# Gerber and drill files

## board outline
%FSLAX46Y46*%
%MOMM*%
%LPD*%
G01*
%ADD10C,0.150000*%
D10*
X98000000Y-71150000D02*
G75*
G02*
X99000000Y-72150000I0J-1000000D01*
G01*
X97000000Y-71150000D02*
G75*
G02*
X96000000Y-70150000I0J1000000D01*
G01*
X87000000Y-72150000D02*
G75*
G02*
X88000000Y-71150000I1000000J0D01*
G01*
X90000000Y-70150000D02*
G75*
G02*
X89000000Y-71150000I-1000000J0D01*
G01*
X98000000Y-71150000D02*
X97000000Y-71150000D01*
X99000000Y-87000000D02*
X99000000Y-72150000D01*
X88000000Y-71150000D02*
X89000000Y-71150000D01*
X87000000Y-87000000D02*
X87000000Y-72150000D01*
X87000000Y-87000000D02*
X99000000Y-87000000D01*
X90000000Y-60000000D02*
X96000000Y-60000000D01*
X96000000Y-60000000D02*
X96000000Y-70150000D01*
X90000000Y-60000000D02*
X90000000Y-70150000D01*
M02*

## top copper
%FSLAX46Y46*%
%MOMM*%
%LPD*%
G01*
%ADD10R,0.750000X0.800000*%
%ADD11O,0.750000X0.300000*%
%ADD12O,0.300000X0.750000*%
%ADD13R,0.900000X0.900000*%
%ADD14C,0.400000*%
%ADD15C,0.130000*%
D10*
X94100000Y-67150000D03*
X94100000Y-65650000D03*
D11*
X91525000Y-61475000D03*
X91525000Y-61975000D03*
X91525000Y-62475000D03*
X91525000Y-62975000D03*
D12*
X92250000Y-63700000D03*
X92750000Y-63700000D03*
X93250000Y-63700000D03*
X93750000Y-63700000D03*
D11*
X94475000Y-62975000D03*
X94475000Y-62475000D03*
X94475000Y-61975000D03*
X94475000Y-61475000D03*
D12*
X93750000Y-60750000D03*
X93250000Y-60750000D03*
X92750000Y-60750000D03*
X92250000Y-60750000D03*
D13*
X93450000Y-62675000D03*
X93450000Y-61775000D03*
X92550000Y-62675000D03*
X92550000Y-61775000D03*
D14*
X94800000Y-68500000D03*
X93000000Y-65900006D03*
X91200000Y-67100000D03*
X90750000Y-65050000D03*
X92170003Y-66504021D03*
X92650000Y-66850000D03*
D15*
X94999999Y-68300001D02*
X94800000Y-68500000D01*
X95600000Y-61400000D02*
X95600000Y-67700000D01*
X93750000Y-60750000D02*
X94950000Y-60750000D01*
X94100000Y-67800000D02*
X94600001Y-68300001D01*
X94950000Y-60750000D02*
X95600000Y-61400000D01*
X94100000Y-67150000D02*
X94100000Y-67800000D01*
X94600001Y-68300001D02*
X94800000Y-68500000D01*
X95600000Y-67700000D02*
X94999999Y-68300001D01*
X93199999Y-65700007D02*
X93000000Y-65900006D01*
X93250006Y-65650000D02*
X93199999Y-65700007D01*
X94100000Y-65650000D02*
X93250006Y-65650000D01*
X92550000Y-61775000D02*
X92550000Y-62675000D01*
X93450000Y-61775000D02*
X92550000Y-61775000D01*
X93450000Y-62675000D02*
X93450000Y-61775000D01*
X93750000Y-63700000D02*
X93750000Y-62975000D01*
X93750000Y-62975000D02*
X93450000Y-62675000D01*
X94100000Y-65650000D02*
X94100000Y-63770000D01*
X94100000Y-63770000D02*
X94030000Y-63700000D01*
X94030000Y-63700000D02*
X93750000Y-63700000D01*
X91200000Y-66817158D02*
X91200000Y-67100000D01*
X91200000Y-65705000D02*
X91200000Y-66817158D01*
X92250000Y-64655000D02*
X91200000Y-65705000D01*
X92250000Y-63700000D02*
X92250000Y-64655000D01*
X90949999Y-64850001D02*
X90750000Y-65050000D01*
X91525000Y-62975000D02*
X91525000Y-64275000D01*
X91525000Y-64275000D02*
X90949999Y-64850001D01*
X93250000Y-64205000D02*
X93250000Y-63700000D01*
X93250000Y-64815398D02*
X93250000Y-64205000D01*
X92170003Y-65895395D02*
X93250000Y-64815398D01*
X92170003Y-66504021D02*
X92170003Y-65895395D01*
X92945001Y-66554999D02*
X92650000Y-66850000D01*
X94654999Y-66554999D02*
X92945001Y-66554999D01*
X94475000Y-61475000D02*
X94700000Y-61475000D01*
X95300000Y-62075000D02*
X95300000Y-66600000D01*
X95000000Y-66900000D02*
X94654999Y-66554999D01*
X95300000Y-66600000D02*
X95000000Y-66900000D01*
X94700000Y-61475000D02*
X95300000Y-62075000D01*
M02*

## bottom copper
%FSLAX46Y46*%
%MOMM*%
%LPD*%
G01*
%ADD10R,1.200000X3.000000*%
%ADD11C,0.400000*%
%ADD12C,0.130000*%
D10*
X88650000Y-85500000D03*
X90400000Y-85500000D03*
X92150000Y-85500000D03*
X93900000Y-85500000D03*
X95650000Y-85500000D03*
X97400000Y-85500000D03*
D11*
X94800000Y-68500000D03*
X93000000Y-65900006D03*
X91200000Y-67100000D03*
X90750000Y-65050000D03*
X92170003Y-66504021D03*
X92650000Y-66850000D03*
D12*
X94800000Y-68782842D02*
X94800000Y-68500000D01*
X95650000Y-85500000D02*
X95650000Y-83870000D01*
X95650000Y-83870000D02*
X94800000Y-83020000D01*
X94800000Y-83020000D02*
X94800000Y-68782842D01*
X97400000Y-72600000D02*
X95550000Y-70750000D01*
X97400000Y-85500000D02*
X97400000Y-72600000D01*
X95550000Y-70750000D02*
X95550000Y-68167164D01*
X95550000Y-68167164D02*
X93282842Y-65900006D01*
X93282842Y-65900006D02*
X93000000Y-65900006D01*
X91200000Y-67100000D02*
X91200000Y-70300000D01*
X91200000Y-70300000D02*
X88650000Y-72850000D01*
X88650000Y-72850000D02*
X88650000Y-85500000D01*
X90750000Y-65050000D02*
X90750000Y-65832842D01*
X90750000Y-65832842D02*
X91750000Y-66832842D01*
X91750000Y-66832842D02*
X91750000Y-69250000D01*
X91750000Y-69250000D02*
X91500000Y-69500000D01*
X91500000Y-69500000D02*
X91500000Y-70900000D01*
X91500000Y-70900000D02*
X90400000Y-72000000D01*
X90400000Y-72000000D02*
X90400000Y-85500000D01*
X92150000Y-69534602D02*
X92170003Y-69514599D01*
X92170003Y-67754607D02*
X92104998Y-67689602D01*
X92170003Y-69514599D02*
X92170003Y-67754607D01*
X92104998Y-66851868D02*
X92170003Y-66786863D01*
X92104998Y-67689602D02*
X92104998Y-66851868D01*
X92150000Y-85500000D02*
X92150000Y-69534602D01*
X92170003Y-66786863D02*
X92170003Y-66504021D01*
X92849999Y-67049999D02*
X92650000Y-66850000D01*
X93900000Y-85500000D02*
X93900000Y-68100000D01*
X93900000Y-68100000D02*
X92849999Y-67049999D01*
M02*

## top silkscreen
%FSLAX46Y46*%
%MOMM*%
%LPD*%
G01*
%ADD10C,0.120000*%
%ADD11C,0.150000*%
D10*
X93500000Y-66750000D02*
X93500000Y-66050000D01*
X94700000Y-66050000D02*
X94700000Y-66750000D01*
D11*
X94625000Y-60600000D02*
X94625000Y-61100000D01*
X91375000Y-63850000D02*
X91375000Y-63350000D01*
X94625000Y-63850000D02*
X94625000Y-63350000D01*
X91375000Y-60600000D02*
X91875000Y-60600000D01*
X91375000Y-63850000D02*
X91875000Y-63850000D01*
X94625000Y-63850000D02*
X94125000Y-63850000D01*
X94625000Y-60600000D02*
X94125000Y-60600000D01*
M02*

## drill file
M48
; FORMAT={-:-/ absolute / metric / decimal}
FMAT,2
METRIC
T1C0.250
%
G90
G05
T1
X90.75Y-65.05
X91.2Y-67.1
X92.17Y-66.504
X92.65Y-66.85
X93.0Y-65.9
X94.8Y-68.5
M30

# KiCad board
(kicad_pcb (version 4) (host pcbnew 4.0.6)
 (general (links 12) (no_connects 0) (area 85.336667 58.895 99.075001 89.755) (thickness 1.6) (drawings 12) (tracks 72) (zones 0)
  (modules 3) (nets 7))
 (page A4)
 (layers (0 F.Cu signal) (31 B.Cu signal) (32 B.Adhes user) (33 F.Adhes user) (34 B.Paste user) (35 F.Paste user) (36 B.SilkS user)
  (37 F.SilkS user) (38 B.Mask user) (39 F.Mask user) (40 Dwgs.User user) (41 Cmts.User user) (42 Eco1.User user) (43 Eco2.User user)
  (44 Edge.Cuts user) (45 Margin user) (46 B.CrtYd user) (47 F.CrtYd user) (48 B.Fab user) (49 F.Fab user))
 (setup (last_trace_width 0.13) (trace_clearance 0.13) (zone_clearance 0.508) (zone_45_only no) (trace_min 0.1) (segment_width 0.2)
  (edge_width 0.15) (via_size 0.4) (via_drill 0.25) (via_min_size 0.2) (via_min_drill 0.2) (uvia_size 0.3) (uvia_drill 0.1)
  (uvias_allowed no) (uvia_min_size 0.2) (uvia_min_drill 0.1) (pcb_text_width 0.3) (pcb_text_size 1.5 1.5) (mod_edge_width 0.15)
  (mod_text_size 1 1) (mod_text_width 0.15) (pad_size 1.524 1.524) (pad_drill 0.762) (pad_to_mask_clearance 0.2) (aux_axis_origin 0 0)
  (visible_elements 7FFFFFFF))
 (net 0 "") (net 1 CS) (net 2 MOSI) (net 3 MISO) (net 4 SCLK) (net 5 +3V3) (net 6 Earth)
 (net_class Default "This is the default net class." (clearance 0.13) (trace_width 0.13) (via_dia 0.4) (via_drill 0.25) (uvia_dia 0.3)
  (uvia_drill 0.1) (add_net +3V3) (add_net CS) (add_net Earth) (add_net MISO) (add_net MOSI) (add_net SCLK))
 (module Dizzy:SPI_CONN (layer B.Cu) (at 90.3 88.25)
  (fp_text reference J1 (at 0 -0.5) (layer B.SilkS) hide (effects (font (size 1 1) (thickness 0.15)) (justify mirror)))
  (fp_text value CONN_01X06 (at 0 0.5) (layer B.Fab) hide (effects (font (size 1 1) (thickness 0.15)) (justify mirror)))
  (pad 1 smd rect (at -1.65 -2.75) (size 1.2 3) (layers B.Cu B.Paste B.Mask) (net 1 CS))
  (pad 2 smd rect (at 0.1 -2.75) (size 1.2 3) (layers B.Cu B.Paste B.Mask) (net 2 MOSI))
  (pad 3 smd rect (at 1.85 -2.75) (size 1.2 3) (layers B.Cu B.Paste B.Mask) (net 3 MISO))
  (pad 4 smd rect (at 3.6 -2.75) (size 1.2 3) (layers B.Cu B.Paste B.Mask) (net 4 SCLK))
  (pad 5 smd rect (at 5.35 -2.75) (size 1.2 3) (layers B.Cu B.Paste B.Mask) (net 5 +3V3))
  (pad 6 smd rect (at 7.1 -2.75) (size 1.2 3) (layers B.Cu B.Paste B.Mask) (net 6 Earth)))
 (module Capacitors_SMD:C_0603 (layer F.Cu) (at 94.1 66.4 270)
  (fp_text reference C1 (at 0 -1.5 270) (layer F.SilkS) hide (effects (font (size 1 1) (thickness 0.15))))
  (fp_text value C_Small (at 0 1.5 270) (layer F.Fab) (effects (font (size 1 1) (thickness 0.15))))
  (fp_line (start 0.35 0.6) (end -0.35 0.6) (layer F.SilkS) (width 0.12))
  (fp_line (start -0.35 -0.6) (end 0.35 -0.6) (layer F.SilkS) (width 0.12))
  (pad 2 smd rect (at 0.75 0 270) (size 0.8 0.75) (layers F.Cu F.Paste F.Mask) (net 5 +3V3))
  (pad 1 smd rect (at -0.75 0 270) (size 0.8 0.75) (layers F.Cu F.Paste F.Mask) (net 6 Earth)))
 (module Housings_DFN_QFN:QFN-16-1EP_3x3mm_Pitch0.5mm (layer F.Cu) (at 93 62.225)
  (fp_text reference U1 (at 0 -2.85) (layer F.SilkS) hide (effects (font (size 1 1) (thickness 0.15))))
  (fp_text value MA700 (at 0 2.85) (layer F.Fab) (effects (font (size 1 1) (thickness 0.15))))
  (fp_line (start 1.625 -1.625) (end 1.625 -1.125) (layer F.SilkS) (width 0.15))
  (fp_line (start -1.625 1.625) (end -1.625 1.125) (layer F.SilkS) (width 0.15))
  (fp_line (start 1.625 1.625) (end 1.625 1.125) (layer F.SilkS) (width 0.15))
  (fp_line (start -1.625 -1.625) (end -1.125 -1.625) (layer F.SilkS) (width 0.15))
  (fp_line (start -1.625 1.625) (end -1.125 1.625) (layer F.SilkS) (width 0.15))
  (fp_line (start 1.625 1.625) (end 1.125 1.625) (layer F.SilkS) (width 0.15))
  (fp_line (start 1.625 -1.625) (end 1.125 -1.625) (layer F.SilkS) (width 0.15))
  (pad 1 smd oval (at -1.475 -0.75) (size 0.75 0.3) (layers F.Cu F.Paste F.Mask))
  (pad 2 smd oval (at -1.475 -0.25) (size 0.75 0.3) (layers F.Cu F.Paste F.Mask))
  (pad 3 smd oval (at -1.475 0.25) (size 0.75 0.3) (layers F.Cu F.Paste F.Mask))
  (pad 4 smd oval (at -1.475 0.75) (size 0.75 0.3) (layers F.Cu F.Paste F.Mask) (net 2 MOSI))
  (pad 5 smd oval (at -0.75 1.475 90) (size 0.75 0.3) (layers F.Cu F.Paste F.Mask) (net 1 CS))
  (pad 6 smd oval (at -0.25 1.475 90) (size 0.75 0.3) (layers F.Cu F.Paste F.Mask))
  (pad 7 smd oval (at 0.25 1.475 90) (size 0.75 0.3) (layers F.Cu F.Paste F.Mask) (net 3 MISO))
  (pad 8 smd oval (at 0.75 1.475 90) (size 0.75 0.3) (layers F.Cu F.Paste F.Mask) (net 6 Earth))
  (pad 9 smd oval (at 1.475 0.75) (size 0.75 0.3) (layers F.Cu F.Paste F.Mask))
  (pad 10 smd oval (at 1.475 0.25) (size 0.75 0.3) (layers F.Cu F.Paste F.Mask))
  (pad 11 smd oval (at 1.475 -0.25) (size 0.75 0.3) (layers F.Cu F.Paste F.Mask))
  (pad 12 smd oval (at 1.475 -0.75) (size 0.75 0.3) (layers F.Cu F.Paste F.Mask) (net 4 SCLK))
  (pad 13 smd oval (at 0.75 -1.475 90) (size 0.75 0.3) (layers F.Cu F.Paste F.Mask) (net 5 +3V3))
  (pad 14 smd oval (at 0.25 -1.475 90) (size 0.75 0.3) (layers F.Cu F.Paste F.Mask))
  (pad 15 smd oval (at -0.25 -1.475 90) (size 0.75 0.3) (layers F.Cu F.Paste F.Mask))
  (pad 16 smd oval (at -0.75 -1.475 90) (size 0.75 0.3) (layers F.Cu F.Paste F.Mask))
  (pad 17 smd rect (at 0.45 0.45) (size 0.9 0.9) (layers F.Cu F.Paste F.Mask) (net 6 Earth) (solder_paste_margin_ratio -0.2))
  (pad 17 smd rect (at 0.45 -0.45) (size 0.9 0.9) (layers F.Cu F.Paste F.Mask) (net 6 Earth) (solder_paste_margin_ratio -0.2))
  (pad 17 smd rect (at -0.45 0.45) (size 0.9 0.9) (layers F.Cu F.Paste F.Mask) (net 6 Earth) (solder_paste_margin_ratio -0.2))
  (pad 17 smd rect (at -0.45 -0.45) (size 0.9 0.9) (layers F.Cu F.Paste F.Mask) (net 6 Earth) (solder_paste_margin_ratio -0.2)))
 (gr_arc (start 98 72.15) (end 98 71.15) (angle 90) (layer Edge.Cuts) (width 0.15))
 (gr_arc (start 97 70.15) (end 97 71.15) (angle 90) (layer Edge.Cuts) (width 0.15))
 (gr_arc (start 88 72.15) (end 87 72.15) (angle 90) (layer Edge.Cuts) (width 0.15))
 (gr_arc (start 89 70.15) (end 90 70.15) (angle 90) (layer Edge.Cuts) (width 0.15))
 (gr_line (start 98 71.15) (end 97 71.15) (layer Edge.Cuts) (width 0.15))
 (gr_line (start 99 87) (end 99 72.15) (layer Edge.Cuts) (width 0.15))
 (gr_line (start 88 71.15) (end 89 71.15) (layer Edge.Cuts) (width 0.15))
 (gr_line (start 87 87) (end 87 72.15) (layer Edge.Cuts) (width 0.15))
 (gr_line (start 87 87) (end 99 87) (layer Edge.Cuts) (width 0.15))
 (gr_line (start 90 60) (end 96 60) (layer Edge.Cuts) (width 0.15))
 (gr_line (start 96 60) (end 96 70.15) (layer Edge.Cuts) (width 0.15))
 (gr_line (start 90 60) (end 90 70.15) (layer Edge.Cuts) (width 0.15))
 (segment (start 94.999999 68.300001) (end 94.8 68.5) (width 0.13) (layer F.Cu) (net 5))
 (segment (start 95.6 61.4) (end 95.6 67.7) (width 0.13) (layer F.Cu) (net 5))
 (segment (start 93.75 60.75) (end 94.95 60.75) (width 0.13) (layer F.Cu) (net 5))
 (segment (start 94.1 67.8) (end 94.600001 68.300001) (width 0.13) (layer F.Cu) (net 5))
 (segment (start 94.95 60.75) (end 95.6 61.4) (width 0.13) (layer F.Cu) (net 5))
 (segment (start 94.1 67.15) (end 94.1 67.8) (width 0.13) (layer F.Cu) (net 5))
 (segment (start 94.600001 68.300001) (end 94.8 68.5) (width 0.13) (layer F.Cu) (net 5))
 (segment (start 94.8 68.782842) (end 94.8 68.5) (width 0.13) (layer B.Cu) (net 5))
 (segment (start 95.6 67.7) (end 94.999999 68.300001) (width 0.13) (layer F.Cu) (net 5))
 (segment (start 95.65 85.5) (end 95.65 83.87) (width 0.13) (layer B.Cu) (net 5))
 (segment (start 95.65 83.87) (end 94.8 83.02) (width 0.13) (layer B.Cu) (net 5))
 (segment (start 94.8 83.02) (end 94.8 68.782842) (width 0.13) (layer B.Cu) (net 5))
 (via (at 94.8 68.5) (size 0.4) (drill 0.25) (layers F.Cu B.Cu) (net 5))
 (segment (start 97.4 72.6) (end 95.55 70.75) (width 0.13) (layer B.Cu) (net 6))
 (segment (start 97.4 85.5) (end 97.4 72.6) (width 0.13) (layer B.Cu) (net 6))
 (segment (start 95.55 70.75) (end 95.55 68.167164) (width 0.13) (layer B.Cu) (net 6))
 (segment (start 95.55 68.167164) (end 93.282842 65.900006) (width 0.13) (layer B.Cu) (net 6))
 (segment (start 93.282842 65.900006) (end 93 65.900006) (width 0.13) (layer B.Cu) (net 6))
 (segment (start 93.199999 65.700007) (end 93 65.900006) (width 0.13) (layer F.Cu) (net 6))
 (segment (start 93.250006 65.65) (end 93.199999 65.700007) (width 0.13) (layer F.Cu) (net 6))
 (segment (start 94.1 65.65) (end 93.250006 65.65) (width 0.13) (layer F.Cu) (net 6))
 (via (at 93 65.900006) (size 0.4) (drill 0.25) (layers F.Cu B.Cu) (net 6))
 (segment (start 92.55 61.775) (end 92.55 62.675) (width 0.13) (layer F.Cu) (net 6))
 (segment (start 93.45 61.775) (end 92.55 61.775) (width 0.13) (layer F.Cu) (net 6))
 (segment (start 93.45 62.675) (end 93.45 61.775) (width 0.13) (layer F.Cu) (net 6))
 (segment (start 93.75 63.7) (end 93.75 62.975) (width 0.13) (layer F.Cu) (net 6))
 (segment (start 93.75 62.975) (end 93.45 62.675) (width 0.13) (layer F.Cu) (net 6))
 (segment (start 94.1 65.65) (end 94.1 63.77) (width 0.13) (layer F.Cu) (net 6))
 (segment (start 94.1 63.77) (end 94.03 63.7) (width 0.13) (layer F.Cu) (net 6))
 (segment (start 94.03 63.7) (end 93.75 63.7) (width 0.13) (layer F.Cu) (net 6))
 (segment (start 91.2 67.1) (end 91.2 70.3) (width 0.13) (layer B.Cu) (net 1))
 (segment (start 91.2 70.3) (end 88.65 72.85) (width 0.13) (layer B.Cu) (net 1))
 (segment (start 88.65 72.85) (end 88.65 85.5) (width 0.13) (layer B.Cu) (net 1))
 (segment (start 91.2 66.817158) (end 91.2 67.1) (width 0.13) (layer F.Cu) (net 1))
 (segment (start 91.2 65.705) (end 91.2 66.817158) (width 0.13) (layer F.Cu) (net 1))
 (segment (start 92.25 64.655) (end 91.2 65.705) (width 0.13) (layer F.Cu) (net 1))
 (via (at 91.2 67.1) (size 0.4) (drill 0.25) (layers F.Cu B.Cu) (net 1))
 (segment (start 92.25 63.7) (end 92.25 64.655) (width 0.13) (layer F.Cu) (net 1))
 (segment (start 90.75 65.05) (end 90.75 65.832842) (width 0.13) (layer B.Cu) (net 2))
 (segment (start 90.75 65.832842) (end 91.75 66.832842) (width 0.13) (layer B.Cu) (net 2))
 (segment (start 91.75 66.832842) (end 91.75 69.25) (width 0.13) (layer B.Cu) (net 2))
 (segment (start 91.75 69.25) (end 91.5 69.5) (width 0.13) (layer B.Cu) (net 2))
 (segment (start 91.5 69.5) (end 91.5 70.9) (width 0.13) (layer B.Cu) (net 2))
 (segment (start 91.5 70.9) (end 90.4 72) (width 0.13) (layer B.Cu) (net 2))
 (segment (start 90.4 72) (end 90.4 85.5) (width 0.13) (layer B.Cu) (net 2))
 (segment (start 90.949999 64.850001) (end 90.75 65.05) (width 0.13) (layer F.Cu) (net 2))
 (segment (start 91.525 62.975) (end 91.525 64.275) (width 0.13) (layer F.Cu) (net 2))
 (segment (start 91.525 64.275) (end 90.949999 64.850001) (width 0.13) (layer F.Cu) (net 2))
 (via (at 90.75 65.05) (size 0.4) (drill 0.25) (layers F.Cu B.Cu) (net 2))
 (segment (start 93.25 64.205) (end 93.25 63.7) (width 0.13) (layer F.Cu) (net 3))
 (segment (start 93.25 64.815398) (end 93.25 64.205) (width 0.13) (layer F.Cu) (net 3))
 (segment (start 92.170003 65.895395) (end 93.25 64.815398) (width 0.13) (layer F.Cu) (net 3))
 (segment (start 92.170003 66.504021) (end 92.170003 65.895395) (width 0.13) (layer F.Cu) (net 3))
 (segment (start 92.15 69.534602) (end 92.170003 69.514599) (width 0.13) (layer B.Cu) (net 3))
 (segment (start 92.170003 67.754607) (end 92.104998 67.689602) (width 0.13) (layer B.Cu) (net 3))
 (segment (start 92.170003 69.514599) (end 92.170003 67.754607) (width 0.13) (layer B.Cu) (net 3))
 (segment (start 92.104998 66.851868) (end 92.170003 66.786863) (width 0.13) (layer B.Cu) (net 3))
 (segment (start 92.104998 67.689602) (end 92.104998 66.851868) (width 0.13) (layer B.Cu) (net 3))
 (segment (start 92.15 85.5) (end 92.15 69.534602) (width 0.13) (layer B.Cu) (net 3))
 (segment (start 92.170003 66.786863) (end 92.170003 66.504021) (width 0.13) (layer B.Cu) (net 3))
 (via (at 92.170003 66.504021) (size 0.4) (drill 0.25) (layers F.Cu B.Cu) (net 3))
 (segment (start 92.945001 66.554999) (end 92.65 66.85) (width 0.13) (layer F.Cu) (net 4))
 (segment (start 94.654999 66.554999) (end 92.945001 66.554999) (width 0.13) (layer F.Cu) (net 4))
 (segment (start 94.475 61.475) (end 94.7 61.475) (width 0.13) (layer F.Cu) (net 4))
 (segment (start 92.849999 67.049999) (end 92.65 66.85) (width 0.13) (layer B.Cu) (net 4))
 (segment (start 93.9 85.5) (end 93.9 68.1) (width 0.13) (layer B.Cu) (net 4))
 (via (at 92.65 66.85) (size 0.4) (drill 0.25) (layers F.Cu B.Cu) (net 4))
 (segment (start 93.9 68.1) (end 92.849999 67.049999) (width 0.13) (layer B.Cu) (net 4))
 (segment (start 95.3 62.075) (end 95.3 66.6) (width 0.13) (layer F.Cu) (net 4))
 (segment (start 95 66.9) (end 94.654999 66.554999) (width 0.13) (layer F.Cu) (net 4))
 (segment (start 95.3 66.6) (end 95 66.9) (width 0.13) (layer F.Cu) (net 4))
 (segment (start 94.7 61.475) (end 95.3 62.075) (width 0.13) (layer F.Cu) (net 4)))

